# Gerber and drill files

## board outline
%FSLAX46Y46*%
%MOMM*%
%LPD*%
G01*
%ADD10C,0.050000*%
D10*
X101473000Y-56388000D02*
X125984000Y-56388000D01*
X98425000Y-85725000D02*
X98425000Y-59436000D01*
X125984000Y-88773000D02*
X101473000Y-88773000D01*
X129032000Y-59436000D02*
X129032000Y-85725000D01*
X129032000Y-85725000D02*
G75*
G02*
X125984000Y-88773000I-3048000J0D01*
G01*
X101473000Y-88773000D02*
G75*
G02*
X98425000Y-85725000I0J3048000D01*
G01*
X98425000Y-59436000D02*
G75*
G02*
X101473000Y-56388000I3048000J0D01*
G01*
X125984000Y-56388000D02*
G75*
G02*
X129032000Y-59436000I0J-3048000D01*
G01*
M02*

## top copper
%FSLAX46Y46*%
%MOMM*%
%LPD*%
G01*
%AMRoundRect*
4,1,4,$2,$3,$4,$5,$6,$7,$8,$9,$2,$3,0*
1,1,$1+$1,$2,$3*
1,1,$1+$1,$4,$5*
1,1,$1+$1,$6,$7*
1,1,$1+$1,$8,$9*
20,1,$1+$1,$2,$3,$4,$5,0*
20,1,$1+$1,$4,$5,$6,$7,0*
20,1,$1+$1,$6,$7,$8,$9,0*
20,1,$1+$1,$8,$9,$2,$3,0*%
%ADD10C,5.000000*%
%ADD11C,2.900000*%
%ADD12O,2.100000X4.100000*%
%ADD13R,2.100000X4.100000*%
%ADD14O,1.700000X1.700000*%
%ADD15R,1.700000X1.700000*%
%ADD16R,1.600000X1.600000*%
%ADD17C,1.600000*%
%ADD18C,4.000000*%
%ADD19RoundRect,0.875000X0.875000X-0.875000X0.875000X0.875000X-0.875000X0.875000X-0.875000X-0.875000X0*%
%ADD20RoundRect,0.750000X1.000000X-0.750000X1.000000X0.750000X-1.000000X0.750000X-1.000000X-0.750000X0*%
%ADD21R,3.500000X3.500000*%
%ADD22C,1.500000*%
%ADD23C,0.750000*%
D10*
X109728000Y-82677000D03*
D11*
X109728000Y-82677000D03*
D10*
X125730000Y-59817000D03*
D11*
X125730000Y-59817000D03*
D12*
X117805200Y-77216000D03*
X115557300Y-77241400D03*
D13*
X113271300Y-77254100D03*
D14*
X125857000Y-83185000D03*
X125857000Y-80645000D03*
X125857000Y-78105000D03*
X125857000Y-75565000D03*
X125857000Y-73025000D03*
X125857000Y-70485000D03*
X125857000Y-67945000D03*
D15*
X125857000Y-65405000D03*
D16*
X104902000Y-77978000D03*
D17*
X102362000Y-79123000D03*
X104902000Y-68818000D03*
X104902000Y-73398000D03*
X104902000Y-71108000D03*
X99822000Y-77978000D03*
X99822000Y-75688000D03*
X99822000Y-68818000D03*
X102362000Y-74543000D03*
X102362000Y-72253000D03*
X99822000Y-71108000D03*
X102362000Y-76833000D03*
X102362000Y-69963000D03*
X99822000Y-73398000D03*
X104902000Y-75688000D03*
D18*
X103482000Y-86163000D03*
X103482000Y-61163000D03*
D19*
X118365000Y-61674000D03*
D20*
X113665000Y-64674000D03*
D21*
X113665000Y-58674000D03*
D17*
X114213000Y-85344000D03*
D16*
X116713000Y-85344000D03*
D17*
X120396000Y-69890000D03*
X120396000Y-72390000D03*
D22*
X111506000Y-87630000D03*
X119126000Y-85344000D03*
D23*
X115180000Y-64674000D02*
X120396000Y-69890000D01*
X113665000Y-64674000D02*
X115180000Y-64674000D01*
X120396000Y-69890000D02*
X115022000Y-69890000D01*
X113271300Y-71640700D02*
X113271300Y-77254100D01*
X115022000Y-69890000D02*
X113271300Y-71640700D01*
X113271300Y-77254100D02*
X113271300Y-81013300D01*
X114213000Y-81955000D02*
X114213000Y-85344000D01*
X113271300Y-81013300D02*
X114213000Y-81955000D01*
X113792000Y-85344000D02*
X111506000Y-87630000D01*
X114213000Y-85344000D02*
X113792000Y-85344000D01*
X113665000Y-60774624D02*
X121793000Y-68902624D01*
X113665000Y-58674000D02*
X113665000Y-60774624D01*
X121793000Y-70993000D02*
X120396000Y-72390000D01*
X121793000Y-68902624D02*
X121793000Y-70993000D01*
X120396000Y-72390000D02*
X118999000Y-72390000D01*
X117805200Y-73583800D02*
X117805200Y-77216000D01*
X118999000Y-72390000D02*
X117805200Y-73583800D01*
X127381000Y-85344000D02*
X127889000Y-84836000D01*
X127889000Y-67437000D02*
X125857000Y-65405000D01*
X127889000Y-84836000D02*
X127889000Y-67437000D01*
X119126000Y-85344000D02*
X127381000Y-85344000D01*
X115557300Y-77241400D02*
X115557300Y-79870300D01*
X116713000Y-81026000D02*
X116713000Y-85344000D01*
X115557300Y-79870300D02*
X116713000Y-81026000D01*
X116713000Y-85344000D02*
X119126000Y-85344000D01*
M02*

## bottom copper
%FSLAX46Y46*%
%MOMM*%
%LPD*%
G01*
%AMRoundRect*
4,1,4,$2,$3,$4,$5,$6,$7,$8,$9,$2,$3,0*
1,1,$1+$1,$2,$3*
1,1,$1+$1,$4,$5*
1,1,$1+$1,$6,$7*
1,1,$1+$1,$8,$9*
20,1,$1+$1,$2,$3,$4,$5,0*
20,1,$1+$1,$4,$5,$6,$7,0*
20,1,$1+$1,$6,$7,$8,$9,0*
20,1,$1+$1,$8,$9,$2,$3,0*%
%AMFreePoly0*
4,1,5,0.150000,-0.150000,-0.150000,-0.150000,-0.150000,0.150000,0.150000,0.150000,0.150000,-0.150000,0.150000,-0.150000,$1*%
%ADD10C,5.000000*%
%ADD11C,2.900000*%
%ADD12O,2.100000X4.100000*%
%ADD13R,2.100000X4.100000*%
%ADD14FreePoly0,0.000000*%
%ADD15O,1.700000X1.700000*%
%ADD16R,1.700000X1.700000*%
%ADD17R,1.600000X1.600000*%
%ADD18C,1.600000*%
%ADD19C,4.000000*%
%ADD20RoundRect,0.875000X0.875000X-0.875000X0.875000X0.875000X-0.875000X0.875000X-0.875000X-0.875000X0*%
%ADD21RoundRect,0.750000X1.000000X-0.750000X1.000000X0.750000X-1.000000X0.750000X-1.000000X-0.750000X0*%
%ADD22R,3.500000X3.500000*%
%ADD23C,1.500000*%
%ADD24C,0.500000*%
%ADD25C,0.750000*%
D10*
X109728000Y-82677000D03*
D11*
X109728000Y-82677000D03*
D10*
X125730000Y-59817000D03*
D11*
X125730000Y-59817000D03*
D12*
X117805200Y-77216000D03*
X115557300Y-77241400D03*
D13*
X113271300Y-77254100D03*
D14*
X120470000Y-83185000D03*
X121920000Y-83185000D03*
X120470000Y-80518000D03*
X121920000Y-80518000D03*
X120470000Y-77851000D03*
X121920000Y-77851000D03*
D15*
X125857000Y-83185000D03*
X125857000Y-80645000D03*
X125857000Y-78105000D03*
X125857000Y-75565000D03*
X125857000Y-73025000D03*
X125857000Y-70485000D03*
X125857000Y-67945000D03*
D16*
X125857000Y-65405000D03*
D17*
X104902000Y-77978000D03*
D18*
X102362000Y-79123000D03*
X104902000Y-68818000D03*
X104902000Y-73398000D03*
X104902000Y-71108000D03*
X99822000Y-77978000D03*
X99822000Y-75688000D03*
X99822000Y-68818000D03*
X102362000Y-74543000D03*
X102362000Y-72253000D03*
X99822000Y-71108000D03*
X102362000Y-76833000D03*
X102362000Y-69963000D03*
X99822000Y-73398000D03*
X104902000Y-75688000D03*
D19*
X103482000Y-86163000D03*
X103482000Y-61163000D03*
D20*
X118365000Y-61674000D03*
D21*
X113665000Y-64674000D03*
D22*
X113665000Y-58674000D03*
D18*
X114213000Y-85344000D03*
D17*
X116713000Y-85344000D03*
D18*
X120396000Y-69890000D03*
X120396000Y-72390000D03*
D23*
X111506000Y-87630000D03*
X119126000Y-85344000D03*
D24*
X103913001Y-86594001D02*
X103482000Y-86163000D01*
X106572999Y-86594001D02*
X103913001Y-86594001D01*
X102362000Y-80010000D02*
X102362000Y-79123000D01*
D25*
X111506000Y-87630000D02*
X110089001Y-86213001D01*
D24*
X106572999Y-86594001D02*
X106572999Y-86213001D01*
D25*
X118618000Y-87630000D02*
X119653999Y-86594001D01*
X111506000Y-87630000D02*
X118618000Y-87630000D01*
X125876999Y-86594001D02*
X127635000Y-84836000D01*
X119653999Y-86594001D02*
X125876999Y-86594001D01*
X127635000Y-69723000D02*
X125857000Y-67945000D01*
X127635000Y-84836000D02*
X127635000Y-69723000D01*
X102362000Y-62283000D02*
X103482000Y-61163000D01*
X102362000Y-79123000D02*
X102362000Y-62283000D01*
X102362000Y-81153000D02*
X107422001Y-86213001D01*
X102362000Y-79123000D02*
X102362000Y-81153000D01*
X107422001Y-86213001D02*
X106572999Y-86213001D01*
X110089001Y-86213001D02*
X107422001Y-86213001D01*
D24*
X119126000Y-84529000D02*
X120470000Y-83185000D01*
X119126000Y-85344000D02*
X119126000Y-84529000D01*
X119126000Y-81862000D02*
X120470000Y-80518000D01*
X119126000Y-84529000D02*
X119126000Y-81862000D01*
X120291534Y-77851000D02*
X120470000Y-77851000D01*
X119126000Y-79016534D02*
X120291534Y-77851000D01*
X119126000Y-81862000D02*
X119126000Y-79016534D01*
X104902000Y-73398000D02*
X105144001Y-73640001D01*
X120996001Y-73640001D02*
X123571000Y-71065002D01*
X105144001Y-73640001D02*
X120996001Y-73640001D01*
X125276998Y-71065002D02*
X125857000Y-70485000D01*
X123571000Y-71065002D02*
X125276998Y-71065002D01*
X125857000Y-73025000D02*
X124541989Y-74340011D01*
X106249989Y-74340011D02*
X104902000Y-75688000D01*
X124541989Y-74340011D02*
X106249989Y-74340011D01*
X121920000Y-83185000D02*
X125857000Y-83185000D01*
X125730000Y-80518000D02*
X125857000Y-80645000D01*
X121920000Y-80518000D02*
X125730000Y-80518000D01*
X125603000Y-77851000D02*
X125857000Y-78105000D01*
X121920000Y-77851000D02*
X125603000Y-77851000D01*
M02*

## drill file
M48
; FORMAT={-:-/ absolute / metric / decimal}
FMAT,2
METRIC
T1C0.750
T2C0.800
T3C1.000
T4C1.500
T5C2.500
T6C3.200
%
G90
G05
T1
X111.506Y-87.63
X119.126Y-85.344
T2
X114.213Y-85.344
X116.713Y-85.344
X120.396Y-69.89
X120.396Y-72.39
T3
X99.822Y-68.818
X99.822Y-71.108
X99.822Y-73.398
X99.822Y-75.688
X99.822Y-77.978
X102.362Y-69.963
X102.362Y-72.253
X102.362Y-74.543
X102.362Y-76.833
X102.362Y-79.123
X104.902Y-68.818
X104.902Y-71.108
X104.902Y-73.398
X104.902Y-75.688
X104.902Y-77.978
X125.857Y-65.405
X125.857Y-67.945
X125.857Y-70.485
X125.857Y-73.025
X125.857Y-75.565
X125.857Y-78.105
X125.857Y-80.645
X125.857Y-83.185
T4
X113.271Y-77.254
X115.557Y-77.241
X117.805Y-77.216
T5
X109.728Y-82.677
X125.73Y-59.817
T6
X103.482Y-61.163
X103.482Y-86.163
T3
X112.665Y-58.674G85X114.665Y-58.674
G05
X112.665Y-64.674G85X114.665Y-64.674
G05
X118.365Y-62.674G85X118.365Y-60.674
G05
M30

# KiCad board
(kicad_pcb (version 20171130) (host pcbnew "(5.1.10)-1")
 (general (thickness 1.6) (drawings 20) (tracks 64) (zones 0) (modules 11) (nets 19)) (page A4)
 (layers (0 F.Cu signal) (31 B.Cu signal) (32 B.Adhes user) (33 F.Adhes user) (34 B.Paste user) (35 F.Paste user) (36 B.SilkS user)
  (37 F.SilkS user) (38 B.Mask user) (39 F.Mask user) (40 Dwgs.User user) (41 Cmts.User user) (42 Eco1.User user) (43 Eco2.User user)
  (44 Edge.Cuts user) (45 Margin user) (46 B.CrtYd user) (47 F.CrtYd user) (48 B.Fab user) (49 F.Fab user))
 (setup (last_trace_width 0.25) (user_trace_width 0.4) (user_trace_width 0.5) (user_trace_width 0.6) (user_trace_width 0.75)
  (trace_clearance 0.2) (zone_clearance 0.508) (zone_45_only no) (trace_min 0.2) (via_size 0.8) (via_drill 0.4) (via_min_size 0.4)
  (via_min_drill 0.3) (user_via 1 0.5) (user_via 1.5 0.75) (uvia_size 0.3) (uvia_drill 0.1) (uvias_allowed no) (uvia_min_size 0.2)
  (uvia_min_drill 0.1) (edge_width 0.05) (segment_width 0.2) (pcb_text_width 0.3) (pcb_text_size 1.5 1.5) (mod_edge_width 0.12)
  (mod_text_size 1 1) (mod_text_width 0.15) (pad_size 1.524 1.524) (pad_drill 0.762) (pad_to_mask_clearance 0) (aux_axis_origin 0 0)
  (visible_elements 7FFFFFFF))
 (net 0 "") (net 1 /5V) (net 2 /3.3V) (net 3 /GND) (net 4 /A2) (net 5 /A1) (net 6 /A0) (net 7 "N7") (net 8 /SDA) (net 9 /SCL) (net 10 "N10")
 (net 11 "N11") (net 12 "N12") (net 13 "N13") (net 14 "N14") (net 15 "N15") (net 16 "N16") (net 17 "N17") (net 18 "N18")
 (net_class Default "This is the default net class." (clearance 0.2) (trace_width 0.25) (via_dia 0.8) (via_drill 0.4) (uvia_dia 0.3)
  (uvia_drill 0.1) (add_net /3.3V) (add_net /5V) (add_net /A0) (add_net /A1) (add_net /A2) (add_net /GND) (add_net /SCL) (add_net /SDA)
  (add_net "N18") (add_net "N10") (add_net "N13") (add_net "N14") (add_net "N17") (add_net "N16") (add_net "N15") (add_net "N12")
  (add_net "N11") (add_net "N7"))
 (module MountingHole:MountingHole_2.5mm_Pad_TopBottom (layer F.Cu) (at 109.728 82.677)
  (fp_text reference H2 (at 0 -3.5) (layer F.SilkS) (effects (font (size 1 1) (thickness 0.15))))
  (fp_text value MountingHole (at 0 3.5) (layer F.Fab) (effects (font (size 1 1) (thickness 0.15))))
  (pad 1 connect circle (at 0 0) (size 5 5) (layers B.Cu B.Mask))
  (pad 1 connect circle (at 0 0) (size 5 5) (layers F.Cu F.Mask))
  (pad 1 thru_hole circle (at 0 0) (size 2.9 2.9) (drill 2.5) (layers *.Cu *.Mask)))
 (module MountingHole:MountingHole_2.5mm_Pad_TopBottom (layer F.Cu) (at 125.73 59.817)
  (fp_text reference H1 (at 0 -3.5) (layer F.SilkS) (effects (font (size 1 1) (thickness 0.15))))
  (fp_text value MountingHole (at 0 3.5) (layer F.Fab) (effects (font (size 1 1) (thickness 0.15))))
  (pad 1 connect circle (at 0 0) (size 5 5) (layers B.Cu B.Mask))
  (pad 1 connect circle (at 0 0) (size 5 5) (layers F.Cu F.Mask))
  (pad 1 thru_hole circle (at 0 0) (size 2.9 2.9) (drill 2.5) (layers *.Cu *.Mask)))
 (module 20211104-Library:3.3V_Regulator (layer F.Cu) (at 110.109 77.216)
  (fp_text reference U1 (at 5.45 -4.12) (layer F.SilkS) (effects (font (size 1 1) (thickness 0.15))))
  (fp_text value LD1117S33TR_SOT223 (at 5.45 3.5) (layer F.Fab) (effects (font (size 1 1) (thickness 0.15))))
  (pad 3 thru_hole oval (at 7.6962 0) (size 2.1 4.1) (drill 1.5) (layers *.Cu *.Mask) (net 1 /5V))
  (pad 2 thru_hole oval (at 5.4483 0.0254) (size 2.1 4.1) (drill 1.5) (layers *.Cu *.Mask) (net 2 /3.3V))
  (pad 1 thru_hole rect (at 3.1623 0.0381) (size 2.1 4.1) (drill 1.5) (layers *.Cu *.Mask) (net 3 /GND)))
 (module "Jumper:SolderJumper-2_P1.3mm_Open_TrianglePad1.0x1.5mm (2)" (layer B.Cu) (at 121.195 83.185)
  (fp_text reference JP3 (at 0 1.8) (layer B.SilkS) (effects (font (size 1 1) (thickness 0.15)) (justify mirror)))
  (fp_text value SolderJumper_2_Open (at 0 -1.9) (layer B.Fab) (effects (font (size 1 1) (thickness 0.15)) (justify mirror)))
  (pad 1 smd custom (at -0.725 0) (size 0.3 0.3) (layers B.Cu B.Mask) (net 2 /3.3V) (zone_connect 2)
   (options (clearance outline) (anchor rect)) (primitives))
  (pad 2 smd custom (at 0.725 0) (size 0.3 0.3) (layers B.Cu B.Mask) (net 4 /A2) (zone_connect 2)
   (options (clearance outline) (anchor rect)) (primitives)))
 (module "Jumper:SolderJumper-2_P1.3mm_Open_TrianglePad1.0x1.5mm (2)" (layer B.Cu) (at 121.195 80.518)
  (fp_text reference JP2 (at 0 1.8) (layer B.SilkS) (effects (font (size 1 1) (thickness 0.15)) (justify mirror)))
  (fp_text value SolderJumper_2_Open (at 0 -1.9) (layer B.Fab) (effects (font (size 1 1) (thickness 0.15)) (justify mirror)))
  (pad 1 smd custom (at -0.725 0) (size 0.3 0.3) (layers B.Cu B.Mask) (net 2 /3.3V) (zone_connect 2)
   (options (clearance outline) (anchor rect)) (primitives))
  (pad 2 smd custom (at 0.725 0) (size 0.3 0.3) (layers B.Cu B.Mask) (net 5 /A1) (zone_connect 2)
   (options (clearance outline) (anchor rect)) (primitives)))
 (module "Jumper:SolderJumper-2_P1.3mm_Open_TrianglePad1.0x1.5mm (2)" (layer B.Cu) (at 121.195 77.851)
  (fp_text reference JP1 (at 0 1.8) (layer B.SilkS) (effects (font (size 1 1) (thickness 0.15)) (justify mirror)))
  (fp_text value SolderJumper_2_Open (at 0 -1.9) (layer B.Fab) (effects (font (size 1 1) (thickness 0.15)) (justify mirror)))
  (pad 1 smd custom (at -0.725 0) (size 0.3 0.3) (layers B.Cu B.Mask) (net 2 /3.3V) (zone_connect 2)
   (options (clearance outline) (anchor rect)) (primitives))
  (pad 2 smd custom (at 0.725 0) (size 0.3 0.3) (layers B.Cu B.Mask) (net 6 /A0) (zone_connect 2)
   (options (clearance outline) (anchor rect)) (primitives)))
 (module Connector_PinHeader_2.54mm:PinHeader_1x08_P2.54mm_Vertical (layer F.Cu) (at 125.857 65.405)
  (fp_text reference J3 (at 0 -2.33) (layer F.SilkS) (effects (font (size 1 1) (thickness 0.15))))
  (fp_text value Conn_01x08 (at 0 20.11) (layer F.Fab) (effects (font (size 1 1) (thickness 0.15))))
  (pad 8 thru_hole oval (at 0 17.78) (size 1.7 1.7) (drill 1) (layers *.Cu *.Mask) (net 4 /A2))
  (pad 7 thru_hole oval (at 0 15.24) (size 1.7 1.7) (drill 1) (layers *.Cu *.Mask) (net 5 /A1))
  (pad 6 thru_hole oval (at 0 12.7) (size 1.7 1.7) (drill 1) (layers *.Cu *.Mask) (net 6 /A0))
  (pad 5 thru_hole oval (at 0 10.16) (size 1.7 1.7) (drill 1) (layers *.Cu *.Mask) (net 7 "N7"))
  (pad 4 thru_hole oval (at 0 7.62) (size 1.7 1.7) (drill 1) (layers *.Cu *.Mask) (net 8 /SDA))
  (pad 3 thru_hole oval (at 0 5.08) (size 1.7 1.7) (drill 1) (layers *.Cu *.Mask) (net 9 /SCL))
  (pad 2 thru_hole oval (at 0 2.54) (size 1.7 1.7) (drill 1) (layers *.Cu *.Mask) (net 3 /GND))
  (pad 1 thru_hole rect (at 0 0) (size 1.7 1.7) (drill 1) (layers *.Cu *.Mask) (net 2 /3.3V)))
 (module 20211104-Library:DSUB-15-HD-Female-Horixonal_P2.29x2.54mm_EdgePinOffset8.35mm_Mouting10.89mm (layer F.Cu) (at 104.902 77.978 270)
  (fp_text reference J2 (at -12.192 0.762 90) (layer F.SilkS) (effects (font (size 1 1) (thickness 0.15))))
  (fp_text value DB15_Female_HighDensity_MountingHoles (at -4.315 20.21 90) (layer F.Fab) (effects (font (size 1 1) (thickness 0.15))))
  (pad 1 thru_hole rect (at 0 0 270) (size 1.6 1.6) (drill 1) (layers *.Cu *.Mask) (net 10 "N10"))
  (pad 6 thru_hole circle (at 1.145 2.54 270) (size 1.6 1.6) (drill 1) (layers *.Cu *.Mask) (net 3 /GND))
  (pad 5 thru_hole circle (at -9.16 0 270) (size 1.6 1.6) (drill 1) (layers *.Cu *.Mask) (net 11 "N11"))
  (pad 3 thru_hole circle (at -4.58 0 270) (size 1.6 1.6) (drill 1) (layers *.Cu *.Mask) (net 9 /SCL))
  (pad 4 thru_hole circle (at -6.87 0 270) (size 1.6 1.6) (drill 1) (layers *.Cu *.Mask) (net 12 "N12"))
  (pad 11 thru_hole circle (at 0 5.08 270) (size 1.6 1.6) (drill 1) (layers *.Cu *.Mask) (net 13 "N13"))
  (pad 12 thru_hole circle (at -2.29 5.08 270) (size 1.6 1.6) (drill 1) (layers *.Cu *.Mask) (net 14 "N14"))
  (pad 15 thru_hole circle (at -9.16 5.08 270) (size 1.6 1.6) (drill 1) (layers *.Cu *.Mask) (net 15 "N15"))
  (pad 8 thru_hole circle (at -3.435 2.54 270) (size 1.6 1.6) (drill 1) (layers *.Cu *.Mask) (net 3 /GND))
  (pad 9 thru_hole circle (at -5.725 2.54 270) (size 1.6 1.6) (drill 1) (layers *.Cu *.Mask) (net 3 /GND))
  (pad 14 thru_hole circle (at -6.87 5.08 270) (size 1.6 1.6) (drill 1) (layers *.Cu *.Mask) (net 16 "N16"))
  (pad 7 thru_hole circle (at -1.145 2.54 270) (size 1.6 1.6) (drill 1) (layers *.Cu *.Mask) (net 3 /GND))
  (pad 10 thru_hole circle (at -8.015 2.54 270) (size 1.6 1.6) (drill 1) (layers *.Cu *.Mask) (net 3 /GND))
  (pad 13 thru_hole circle (at -4.58 5.08 270) (size 1.6 1.6) (drill 1) (layers *.Cu *.Mask) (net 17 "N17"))
  (pad 2 thru_hole circle (at -2.29 0 270) (size 1.6 1.6) (drill 1) (layers *.Cu *.Mask) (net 8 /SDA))
  (pad 0 thru_hole circle (at 8.185 1.42 270) (size 4 4) (drill 3.2) (layers *.Cu *.Mask) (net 3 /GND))
  (pad 0 thru_hole circle (at -16.815 1.42 270) (size 4 4) (drill 3.2) (layers *.Cu *.Mask) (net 3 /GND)))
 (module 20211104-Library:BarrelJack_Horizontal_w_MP (layer F.Cu) (at 113.665 58.674 90)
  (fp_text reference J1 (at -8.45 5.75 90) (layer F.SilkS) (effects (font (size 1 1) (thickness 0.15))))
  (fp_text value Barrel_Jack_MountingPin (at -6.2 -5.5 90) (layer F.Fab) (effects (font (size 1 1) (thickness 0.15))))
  (pad MP thru_hole roundrect (at -3 4.7 90) (size 3.5 3.5) (drill oval 3 1) (layers *.Cu *.Mask) (roundrect_rratio 0.25) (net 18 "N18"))
  (pad 2 thru_hole roundrect (at -6 0 90) (size 3 3.5) (drill oval 1 3) (layers *.Cu *.Mask) (roundrect_rratio 0.25) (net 3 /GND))
  (pad 1 thru_hole rect (at 0 0 90) (size 3.5 3.5) (drill oval 1 3) (layers *.Cu *.Mask) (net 1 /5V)))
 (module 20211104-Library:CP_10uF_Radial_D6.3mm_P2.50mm (layer F.Cu) (at 116.713 85.344 180)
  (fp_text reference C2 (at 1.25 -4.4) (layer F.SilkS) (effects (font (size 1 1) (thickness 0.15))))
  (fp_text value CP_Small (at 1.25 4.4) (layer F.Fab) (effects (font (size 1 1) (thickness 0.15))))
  (pad 2 thru_hole circle (at 2.5 0 180) (size 1.6 1.6) (drill 0.8) (layers *.Cu *.Mask) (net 3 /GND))
  (pad 1 thru_hole rect (at 0 0 180) (size 1.6 1.6) (drill 0.8) (layers *.Cu *.Mask) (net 2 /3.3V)))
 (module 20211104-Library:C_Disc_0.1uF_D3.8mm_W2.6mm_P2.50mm (layer F.Cu) (at 120.396 72.39 90)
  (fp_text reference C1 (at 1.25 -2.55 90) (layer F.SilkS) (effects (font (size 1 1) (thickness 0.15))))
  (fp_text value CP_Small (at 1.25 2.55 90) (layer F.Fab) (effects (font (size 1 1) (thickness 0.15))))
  (pad 2 thru_hole circle (at 2.5 0 90) (size 1.6 1.6) (drill 0.8) (layers *.Cu *.Mask) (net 3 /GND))
  (pad 1 thru_hole circle (at 0 0 90) (size 1.6 1.6) (drill 0.8) (layers *.Cu *.Mask) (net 1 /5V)))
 (gr_line (start 101.473 56.388) (end 125.984 56.388) (layer Edge.Cuts) (width 0.05))
 (gr_line (start 98.425 85.725) (end 98.425 59.436) (layer Edge.Cuts) (width 0.05))
 (gr_line (start 125.984 88.773) (end 101.473 88.773) (layer Edge.Cuts) (width 0.05))
 (gr_line (start 129.032 59.436) (end 129.032 85.725) (layer Edge.Cuts) (width 0.05))
 (gr_arc (start 125.984 85.725) (end 125.984 88.773) (angle -90) (layer Edge.Cuts) (width 0.05))
 (gr_arc (start 101.473 85.725) (end 98.425 85.725) (angle -90) (layer Edge.Cuts) (width 0.05))
 (gr_arc (start 101.473 59.436) (end 101.473 56.388) (angle -90) (layer Edge.Cuts) (width 0.05))
 (gr_arc (start 125.984 59.436) (end 129.032 59.436) (angle -90) (layer Edge.Cuts) (width 0.05))
 (segment (start 115.18 64.674) (end 120.396 69.89) (width 0.75) (layer F.Cu) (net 3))
 (segment (start 113.665 64.674) (end 115.18 64.674) (width 0.75) (layer F.Cu) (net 3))
 (segment (start 120.396 69.89) (end 115.022 69.89) (width 0.75) (layer F.Cu) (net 3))
 (segment (start 113.2713 71.6407) (end 113.2713 77.2541) (width 0.75) (layer F.Cu) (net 3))
 (segment (start 115.022 69.89) (end 113.2713 71.6407) (width 0.75) (layer F.Cu) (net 3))
 (segment (start 103.913001 86.594001) (end 103.482 86.163) (width 0.5) (layer B.Cu) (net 3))
 (segment (start 106.572999 86.594001) (end 103.913001 86.594001) (width 0.5) (layer B.Cu) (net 3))
 (segment (start 102.362 80.01) (end 102.362 79.123) (width 0.5) (layer B.Cu) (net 3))
 (segment (start 113.2713 77.2541) (end 113.2713 81.0133) (width 0.75) (layer F.Cu) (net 3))
 (segment (start 114.213 81.955) (end 114.213 85.344) (width 0.75) (layer F.Cu) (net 3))
 (segment (start 113.2713 81.0133) (end 114.213 81.955) (width 0.75) (layer F.Cu) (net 3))
 (via (at 111.506 87.63) (size 1.5) (drill 0.75) (layers F.Cu B.Cu) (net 3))
 (segment (start 113.792 85.344) (end 111.506 87.63) (width 0.75) (layer F.Cu) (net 3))
 (segment (start 114.213 85.344) (end 113.792 85.344) (width 0.75) (layer F.Cu) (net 3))
 (segment (start 111.506 87.63) (end 110.089001 86.213001) (width 0.75) (layer B.Cu) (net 3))
 (segment (start 106.572999 86.594001) (end 106.572999 86.213001) (width 0.5) (layer B.Cu) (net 3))
 (segment (start 118.618 87.63) (end 119.653999 86.594001) (width 0.75) (layer B.Cu) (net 3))
 (segment (start 111.506 87.63) (end 118.618 87.63) (width 0.75) (layer B.Cu) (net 3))
 (segment (start 125.876999 86.594001) (end 127.635 84.836) (width 0.75) (layer B.Cu) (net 3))
 (segment (start 119.653999 86.594001) (end 125.876999 86.594001) (width 0.75) (layer B.Cu) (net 3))
 (segment (start 127.635 69.723) (end 125.857 67.945) (width 0.75) (layer B.Cu) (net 3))
 (segment (start 127.635 84.836) (end 127.635 69.723) (width 0.75) (layer B.Cu) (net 3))
 (segment (start 102.362 62.283) (end 103.482 61.163) (width 0.75) (layer B.Cu) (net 3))
 (segment (start 102.362 79.123) (end 102.362 62.283) (width 0.75) (layer B.Cu) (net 3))
 (segment (start 102.362 81.153) (end 107.422001 86.213001) (width 0.75) (layer B.Cu) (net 3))
 (segment (start 102.362 79.123) (end 102.362 81.153) (width 0.75) (layer B.Cu) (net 3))
 (segment (start 107.422001 86.213001) (end 106.572999 86.213001) (width 0.75) (layer B.Cu) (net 3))
 (segment (start 110.089001 86.213001) (end 107.422001 86.213001) (width 0.75) (layer B.Cu) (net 3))
 (segment (start 113.665 60.774624) (end 121.793 68.902624) (width 0.75) (layer F.Cu) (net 1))
 (segment (start 113.665 58.674) (end 113.665 60.774624) (width 0.75) (layer F.Cu) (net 1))
 (segment (start 121.793 70.993) (end 120.396 72.39) (width 0.75) (layer F.Cu) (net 1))
 (segment (start 121.793 68.902624) (end 121.793 70.993) (width 0.75) (layer F.Cu) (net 1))
 (segment (start 120.396 72.39) (end 118.999 72.39) (width 0.75) (layer F.Cu) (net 1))
 (segment (start 117.8052 73.5838) (end 117.8052 77.216) (width 0.75) (layer F.Cu) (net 1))
 (segment (start 118.999 72.39) (end 117.8052 73.5838) (width 0.75) (layer F.Cu) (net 1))
 (segment (start 127.381 85.344) (end 127.889 84.836) (width 0.75) (layer F.Cu) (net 2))
 (segment (start 127.889 67.437) (end 125.857 65.405) (width 0.75) (layer F.Cu) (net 2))
 (segment (start 127.889 84.836) (end 127.889 67.437) (width 0.75) (layer F.Cu) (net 2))
 (segment (start 119.126 85.344) (end 127.381 85.344) (width 0.75) (layer F.Cu) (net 2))
 (via (at 119.126 85.344) (size 1.5) (drill 0.75) (layers F.Cu B.Cu) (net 2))
 (segment (start 119.126 84.529) (end 120.47 83.185) (width 0.5) (layer B.Cu) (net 2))
 (segment (start 119.126 85.344) (end 119.126 84.529) (width 0.5) (layer B.Cu) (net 2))
 (segment (start 119.126 81.862) (end 120.47 80.518) (width 0.5) (layer B.Cu) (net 2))
 (segment (start 119.126 84.529) (end 119.126 81.862) (width 0.5) (layer B.Cu) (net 2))
 (segment (start 120.291534 77.851) (end 120.47 77.851) (width 0.5) (layer B.Cu) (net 2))
 (segment (start 119.126 79.016534) (end 120.291534 77.851) (width 0.5) (layer B.Cu) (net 2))
 (segment (start 119.126 81.862) (end 119.126 79.016534) (width 0.5) (layer B.Cu) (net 2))
 (segment (start 115.5573 77.2414) (end 115.5573 79.8703) (width 0.75) (layer F.Cu) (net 2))
 (segment (start 116.713 81.026) (end 116.713 85.344) (width 0.75) (layer F.Cu) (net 2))
 (segment (start 115.5573 79.8703) (end 116.713 81.026) (width 0.75) (layer F.Cu) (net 2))
 (segment (start 116.713 85.344) (end 119.126 85.344) (width 0.75) (layer F.Cu) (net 2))
 (segment (start 104.902 73.398) (end 105.144001 73.640001) (width 0.5) (layer B.Cu) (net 9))
 (segment (start 120.996001 73.640001) (end 123.571 71.065002) (width 0.5) (layer B.Cu) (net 9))
 (segment (start 105.144001 73.640001) (end 120.996001 73.640001) (width 0.5) (layer B.Cu) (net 9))
 (segment (start 125.276998 71.065002) (end 125.857 70.485) (width 0.5) (layer B.Cu) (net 9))
 (segment (start 123.571 71.065002) (end 125.276998 71.065002) (width 0.5) (layer B.Cu) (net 9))
 (segment (start 125.857 73.025) (end 124.541989 74.340011) (width 0.5) (layer B.Cu) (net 8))
 (segment (start 106.249989 74.340011) (end 104.902 75.688) (width 0.5) (layer B.Cu) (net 8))
 (segment (start 124.541989 74.340011) (end 106.249989 74.340011) (width 0.5) (layer B.Cu) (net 8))
 (segment (start 121.92 83.185) (end 125.857 83.185) (width 0.5) (layer B.Cu) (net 4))
 (segment (start 125.73 80.518) (end 125.857 80.645) (width 0.5) (layer B.Cu) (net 5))
 (segment (start 121.92 80.518) (end 125.73 80.518) (width 0.5) (layer B.Cu) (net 5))
 (segment (start 125.603 77.851) (end 125.857 78.105) (width 0.5) (layer B.Cu) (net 6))
 (segment (start 121.92 77.851) (end 125.603 77.851) (width 0.5) (layer B.Cu) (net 6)))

